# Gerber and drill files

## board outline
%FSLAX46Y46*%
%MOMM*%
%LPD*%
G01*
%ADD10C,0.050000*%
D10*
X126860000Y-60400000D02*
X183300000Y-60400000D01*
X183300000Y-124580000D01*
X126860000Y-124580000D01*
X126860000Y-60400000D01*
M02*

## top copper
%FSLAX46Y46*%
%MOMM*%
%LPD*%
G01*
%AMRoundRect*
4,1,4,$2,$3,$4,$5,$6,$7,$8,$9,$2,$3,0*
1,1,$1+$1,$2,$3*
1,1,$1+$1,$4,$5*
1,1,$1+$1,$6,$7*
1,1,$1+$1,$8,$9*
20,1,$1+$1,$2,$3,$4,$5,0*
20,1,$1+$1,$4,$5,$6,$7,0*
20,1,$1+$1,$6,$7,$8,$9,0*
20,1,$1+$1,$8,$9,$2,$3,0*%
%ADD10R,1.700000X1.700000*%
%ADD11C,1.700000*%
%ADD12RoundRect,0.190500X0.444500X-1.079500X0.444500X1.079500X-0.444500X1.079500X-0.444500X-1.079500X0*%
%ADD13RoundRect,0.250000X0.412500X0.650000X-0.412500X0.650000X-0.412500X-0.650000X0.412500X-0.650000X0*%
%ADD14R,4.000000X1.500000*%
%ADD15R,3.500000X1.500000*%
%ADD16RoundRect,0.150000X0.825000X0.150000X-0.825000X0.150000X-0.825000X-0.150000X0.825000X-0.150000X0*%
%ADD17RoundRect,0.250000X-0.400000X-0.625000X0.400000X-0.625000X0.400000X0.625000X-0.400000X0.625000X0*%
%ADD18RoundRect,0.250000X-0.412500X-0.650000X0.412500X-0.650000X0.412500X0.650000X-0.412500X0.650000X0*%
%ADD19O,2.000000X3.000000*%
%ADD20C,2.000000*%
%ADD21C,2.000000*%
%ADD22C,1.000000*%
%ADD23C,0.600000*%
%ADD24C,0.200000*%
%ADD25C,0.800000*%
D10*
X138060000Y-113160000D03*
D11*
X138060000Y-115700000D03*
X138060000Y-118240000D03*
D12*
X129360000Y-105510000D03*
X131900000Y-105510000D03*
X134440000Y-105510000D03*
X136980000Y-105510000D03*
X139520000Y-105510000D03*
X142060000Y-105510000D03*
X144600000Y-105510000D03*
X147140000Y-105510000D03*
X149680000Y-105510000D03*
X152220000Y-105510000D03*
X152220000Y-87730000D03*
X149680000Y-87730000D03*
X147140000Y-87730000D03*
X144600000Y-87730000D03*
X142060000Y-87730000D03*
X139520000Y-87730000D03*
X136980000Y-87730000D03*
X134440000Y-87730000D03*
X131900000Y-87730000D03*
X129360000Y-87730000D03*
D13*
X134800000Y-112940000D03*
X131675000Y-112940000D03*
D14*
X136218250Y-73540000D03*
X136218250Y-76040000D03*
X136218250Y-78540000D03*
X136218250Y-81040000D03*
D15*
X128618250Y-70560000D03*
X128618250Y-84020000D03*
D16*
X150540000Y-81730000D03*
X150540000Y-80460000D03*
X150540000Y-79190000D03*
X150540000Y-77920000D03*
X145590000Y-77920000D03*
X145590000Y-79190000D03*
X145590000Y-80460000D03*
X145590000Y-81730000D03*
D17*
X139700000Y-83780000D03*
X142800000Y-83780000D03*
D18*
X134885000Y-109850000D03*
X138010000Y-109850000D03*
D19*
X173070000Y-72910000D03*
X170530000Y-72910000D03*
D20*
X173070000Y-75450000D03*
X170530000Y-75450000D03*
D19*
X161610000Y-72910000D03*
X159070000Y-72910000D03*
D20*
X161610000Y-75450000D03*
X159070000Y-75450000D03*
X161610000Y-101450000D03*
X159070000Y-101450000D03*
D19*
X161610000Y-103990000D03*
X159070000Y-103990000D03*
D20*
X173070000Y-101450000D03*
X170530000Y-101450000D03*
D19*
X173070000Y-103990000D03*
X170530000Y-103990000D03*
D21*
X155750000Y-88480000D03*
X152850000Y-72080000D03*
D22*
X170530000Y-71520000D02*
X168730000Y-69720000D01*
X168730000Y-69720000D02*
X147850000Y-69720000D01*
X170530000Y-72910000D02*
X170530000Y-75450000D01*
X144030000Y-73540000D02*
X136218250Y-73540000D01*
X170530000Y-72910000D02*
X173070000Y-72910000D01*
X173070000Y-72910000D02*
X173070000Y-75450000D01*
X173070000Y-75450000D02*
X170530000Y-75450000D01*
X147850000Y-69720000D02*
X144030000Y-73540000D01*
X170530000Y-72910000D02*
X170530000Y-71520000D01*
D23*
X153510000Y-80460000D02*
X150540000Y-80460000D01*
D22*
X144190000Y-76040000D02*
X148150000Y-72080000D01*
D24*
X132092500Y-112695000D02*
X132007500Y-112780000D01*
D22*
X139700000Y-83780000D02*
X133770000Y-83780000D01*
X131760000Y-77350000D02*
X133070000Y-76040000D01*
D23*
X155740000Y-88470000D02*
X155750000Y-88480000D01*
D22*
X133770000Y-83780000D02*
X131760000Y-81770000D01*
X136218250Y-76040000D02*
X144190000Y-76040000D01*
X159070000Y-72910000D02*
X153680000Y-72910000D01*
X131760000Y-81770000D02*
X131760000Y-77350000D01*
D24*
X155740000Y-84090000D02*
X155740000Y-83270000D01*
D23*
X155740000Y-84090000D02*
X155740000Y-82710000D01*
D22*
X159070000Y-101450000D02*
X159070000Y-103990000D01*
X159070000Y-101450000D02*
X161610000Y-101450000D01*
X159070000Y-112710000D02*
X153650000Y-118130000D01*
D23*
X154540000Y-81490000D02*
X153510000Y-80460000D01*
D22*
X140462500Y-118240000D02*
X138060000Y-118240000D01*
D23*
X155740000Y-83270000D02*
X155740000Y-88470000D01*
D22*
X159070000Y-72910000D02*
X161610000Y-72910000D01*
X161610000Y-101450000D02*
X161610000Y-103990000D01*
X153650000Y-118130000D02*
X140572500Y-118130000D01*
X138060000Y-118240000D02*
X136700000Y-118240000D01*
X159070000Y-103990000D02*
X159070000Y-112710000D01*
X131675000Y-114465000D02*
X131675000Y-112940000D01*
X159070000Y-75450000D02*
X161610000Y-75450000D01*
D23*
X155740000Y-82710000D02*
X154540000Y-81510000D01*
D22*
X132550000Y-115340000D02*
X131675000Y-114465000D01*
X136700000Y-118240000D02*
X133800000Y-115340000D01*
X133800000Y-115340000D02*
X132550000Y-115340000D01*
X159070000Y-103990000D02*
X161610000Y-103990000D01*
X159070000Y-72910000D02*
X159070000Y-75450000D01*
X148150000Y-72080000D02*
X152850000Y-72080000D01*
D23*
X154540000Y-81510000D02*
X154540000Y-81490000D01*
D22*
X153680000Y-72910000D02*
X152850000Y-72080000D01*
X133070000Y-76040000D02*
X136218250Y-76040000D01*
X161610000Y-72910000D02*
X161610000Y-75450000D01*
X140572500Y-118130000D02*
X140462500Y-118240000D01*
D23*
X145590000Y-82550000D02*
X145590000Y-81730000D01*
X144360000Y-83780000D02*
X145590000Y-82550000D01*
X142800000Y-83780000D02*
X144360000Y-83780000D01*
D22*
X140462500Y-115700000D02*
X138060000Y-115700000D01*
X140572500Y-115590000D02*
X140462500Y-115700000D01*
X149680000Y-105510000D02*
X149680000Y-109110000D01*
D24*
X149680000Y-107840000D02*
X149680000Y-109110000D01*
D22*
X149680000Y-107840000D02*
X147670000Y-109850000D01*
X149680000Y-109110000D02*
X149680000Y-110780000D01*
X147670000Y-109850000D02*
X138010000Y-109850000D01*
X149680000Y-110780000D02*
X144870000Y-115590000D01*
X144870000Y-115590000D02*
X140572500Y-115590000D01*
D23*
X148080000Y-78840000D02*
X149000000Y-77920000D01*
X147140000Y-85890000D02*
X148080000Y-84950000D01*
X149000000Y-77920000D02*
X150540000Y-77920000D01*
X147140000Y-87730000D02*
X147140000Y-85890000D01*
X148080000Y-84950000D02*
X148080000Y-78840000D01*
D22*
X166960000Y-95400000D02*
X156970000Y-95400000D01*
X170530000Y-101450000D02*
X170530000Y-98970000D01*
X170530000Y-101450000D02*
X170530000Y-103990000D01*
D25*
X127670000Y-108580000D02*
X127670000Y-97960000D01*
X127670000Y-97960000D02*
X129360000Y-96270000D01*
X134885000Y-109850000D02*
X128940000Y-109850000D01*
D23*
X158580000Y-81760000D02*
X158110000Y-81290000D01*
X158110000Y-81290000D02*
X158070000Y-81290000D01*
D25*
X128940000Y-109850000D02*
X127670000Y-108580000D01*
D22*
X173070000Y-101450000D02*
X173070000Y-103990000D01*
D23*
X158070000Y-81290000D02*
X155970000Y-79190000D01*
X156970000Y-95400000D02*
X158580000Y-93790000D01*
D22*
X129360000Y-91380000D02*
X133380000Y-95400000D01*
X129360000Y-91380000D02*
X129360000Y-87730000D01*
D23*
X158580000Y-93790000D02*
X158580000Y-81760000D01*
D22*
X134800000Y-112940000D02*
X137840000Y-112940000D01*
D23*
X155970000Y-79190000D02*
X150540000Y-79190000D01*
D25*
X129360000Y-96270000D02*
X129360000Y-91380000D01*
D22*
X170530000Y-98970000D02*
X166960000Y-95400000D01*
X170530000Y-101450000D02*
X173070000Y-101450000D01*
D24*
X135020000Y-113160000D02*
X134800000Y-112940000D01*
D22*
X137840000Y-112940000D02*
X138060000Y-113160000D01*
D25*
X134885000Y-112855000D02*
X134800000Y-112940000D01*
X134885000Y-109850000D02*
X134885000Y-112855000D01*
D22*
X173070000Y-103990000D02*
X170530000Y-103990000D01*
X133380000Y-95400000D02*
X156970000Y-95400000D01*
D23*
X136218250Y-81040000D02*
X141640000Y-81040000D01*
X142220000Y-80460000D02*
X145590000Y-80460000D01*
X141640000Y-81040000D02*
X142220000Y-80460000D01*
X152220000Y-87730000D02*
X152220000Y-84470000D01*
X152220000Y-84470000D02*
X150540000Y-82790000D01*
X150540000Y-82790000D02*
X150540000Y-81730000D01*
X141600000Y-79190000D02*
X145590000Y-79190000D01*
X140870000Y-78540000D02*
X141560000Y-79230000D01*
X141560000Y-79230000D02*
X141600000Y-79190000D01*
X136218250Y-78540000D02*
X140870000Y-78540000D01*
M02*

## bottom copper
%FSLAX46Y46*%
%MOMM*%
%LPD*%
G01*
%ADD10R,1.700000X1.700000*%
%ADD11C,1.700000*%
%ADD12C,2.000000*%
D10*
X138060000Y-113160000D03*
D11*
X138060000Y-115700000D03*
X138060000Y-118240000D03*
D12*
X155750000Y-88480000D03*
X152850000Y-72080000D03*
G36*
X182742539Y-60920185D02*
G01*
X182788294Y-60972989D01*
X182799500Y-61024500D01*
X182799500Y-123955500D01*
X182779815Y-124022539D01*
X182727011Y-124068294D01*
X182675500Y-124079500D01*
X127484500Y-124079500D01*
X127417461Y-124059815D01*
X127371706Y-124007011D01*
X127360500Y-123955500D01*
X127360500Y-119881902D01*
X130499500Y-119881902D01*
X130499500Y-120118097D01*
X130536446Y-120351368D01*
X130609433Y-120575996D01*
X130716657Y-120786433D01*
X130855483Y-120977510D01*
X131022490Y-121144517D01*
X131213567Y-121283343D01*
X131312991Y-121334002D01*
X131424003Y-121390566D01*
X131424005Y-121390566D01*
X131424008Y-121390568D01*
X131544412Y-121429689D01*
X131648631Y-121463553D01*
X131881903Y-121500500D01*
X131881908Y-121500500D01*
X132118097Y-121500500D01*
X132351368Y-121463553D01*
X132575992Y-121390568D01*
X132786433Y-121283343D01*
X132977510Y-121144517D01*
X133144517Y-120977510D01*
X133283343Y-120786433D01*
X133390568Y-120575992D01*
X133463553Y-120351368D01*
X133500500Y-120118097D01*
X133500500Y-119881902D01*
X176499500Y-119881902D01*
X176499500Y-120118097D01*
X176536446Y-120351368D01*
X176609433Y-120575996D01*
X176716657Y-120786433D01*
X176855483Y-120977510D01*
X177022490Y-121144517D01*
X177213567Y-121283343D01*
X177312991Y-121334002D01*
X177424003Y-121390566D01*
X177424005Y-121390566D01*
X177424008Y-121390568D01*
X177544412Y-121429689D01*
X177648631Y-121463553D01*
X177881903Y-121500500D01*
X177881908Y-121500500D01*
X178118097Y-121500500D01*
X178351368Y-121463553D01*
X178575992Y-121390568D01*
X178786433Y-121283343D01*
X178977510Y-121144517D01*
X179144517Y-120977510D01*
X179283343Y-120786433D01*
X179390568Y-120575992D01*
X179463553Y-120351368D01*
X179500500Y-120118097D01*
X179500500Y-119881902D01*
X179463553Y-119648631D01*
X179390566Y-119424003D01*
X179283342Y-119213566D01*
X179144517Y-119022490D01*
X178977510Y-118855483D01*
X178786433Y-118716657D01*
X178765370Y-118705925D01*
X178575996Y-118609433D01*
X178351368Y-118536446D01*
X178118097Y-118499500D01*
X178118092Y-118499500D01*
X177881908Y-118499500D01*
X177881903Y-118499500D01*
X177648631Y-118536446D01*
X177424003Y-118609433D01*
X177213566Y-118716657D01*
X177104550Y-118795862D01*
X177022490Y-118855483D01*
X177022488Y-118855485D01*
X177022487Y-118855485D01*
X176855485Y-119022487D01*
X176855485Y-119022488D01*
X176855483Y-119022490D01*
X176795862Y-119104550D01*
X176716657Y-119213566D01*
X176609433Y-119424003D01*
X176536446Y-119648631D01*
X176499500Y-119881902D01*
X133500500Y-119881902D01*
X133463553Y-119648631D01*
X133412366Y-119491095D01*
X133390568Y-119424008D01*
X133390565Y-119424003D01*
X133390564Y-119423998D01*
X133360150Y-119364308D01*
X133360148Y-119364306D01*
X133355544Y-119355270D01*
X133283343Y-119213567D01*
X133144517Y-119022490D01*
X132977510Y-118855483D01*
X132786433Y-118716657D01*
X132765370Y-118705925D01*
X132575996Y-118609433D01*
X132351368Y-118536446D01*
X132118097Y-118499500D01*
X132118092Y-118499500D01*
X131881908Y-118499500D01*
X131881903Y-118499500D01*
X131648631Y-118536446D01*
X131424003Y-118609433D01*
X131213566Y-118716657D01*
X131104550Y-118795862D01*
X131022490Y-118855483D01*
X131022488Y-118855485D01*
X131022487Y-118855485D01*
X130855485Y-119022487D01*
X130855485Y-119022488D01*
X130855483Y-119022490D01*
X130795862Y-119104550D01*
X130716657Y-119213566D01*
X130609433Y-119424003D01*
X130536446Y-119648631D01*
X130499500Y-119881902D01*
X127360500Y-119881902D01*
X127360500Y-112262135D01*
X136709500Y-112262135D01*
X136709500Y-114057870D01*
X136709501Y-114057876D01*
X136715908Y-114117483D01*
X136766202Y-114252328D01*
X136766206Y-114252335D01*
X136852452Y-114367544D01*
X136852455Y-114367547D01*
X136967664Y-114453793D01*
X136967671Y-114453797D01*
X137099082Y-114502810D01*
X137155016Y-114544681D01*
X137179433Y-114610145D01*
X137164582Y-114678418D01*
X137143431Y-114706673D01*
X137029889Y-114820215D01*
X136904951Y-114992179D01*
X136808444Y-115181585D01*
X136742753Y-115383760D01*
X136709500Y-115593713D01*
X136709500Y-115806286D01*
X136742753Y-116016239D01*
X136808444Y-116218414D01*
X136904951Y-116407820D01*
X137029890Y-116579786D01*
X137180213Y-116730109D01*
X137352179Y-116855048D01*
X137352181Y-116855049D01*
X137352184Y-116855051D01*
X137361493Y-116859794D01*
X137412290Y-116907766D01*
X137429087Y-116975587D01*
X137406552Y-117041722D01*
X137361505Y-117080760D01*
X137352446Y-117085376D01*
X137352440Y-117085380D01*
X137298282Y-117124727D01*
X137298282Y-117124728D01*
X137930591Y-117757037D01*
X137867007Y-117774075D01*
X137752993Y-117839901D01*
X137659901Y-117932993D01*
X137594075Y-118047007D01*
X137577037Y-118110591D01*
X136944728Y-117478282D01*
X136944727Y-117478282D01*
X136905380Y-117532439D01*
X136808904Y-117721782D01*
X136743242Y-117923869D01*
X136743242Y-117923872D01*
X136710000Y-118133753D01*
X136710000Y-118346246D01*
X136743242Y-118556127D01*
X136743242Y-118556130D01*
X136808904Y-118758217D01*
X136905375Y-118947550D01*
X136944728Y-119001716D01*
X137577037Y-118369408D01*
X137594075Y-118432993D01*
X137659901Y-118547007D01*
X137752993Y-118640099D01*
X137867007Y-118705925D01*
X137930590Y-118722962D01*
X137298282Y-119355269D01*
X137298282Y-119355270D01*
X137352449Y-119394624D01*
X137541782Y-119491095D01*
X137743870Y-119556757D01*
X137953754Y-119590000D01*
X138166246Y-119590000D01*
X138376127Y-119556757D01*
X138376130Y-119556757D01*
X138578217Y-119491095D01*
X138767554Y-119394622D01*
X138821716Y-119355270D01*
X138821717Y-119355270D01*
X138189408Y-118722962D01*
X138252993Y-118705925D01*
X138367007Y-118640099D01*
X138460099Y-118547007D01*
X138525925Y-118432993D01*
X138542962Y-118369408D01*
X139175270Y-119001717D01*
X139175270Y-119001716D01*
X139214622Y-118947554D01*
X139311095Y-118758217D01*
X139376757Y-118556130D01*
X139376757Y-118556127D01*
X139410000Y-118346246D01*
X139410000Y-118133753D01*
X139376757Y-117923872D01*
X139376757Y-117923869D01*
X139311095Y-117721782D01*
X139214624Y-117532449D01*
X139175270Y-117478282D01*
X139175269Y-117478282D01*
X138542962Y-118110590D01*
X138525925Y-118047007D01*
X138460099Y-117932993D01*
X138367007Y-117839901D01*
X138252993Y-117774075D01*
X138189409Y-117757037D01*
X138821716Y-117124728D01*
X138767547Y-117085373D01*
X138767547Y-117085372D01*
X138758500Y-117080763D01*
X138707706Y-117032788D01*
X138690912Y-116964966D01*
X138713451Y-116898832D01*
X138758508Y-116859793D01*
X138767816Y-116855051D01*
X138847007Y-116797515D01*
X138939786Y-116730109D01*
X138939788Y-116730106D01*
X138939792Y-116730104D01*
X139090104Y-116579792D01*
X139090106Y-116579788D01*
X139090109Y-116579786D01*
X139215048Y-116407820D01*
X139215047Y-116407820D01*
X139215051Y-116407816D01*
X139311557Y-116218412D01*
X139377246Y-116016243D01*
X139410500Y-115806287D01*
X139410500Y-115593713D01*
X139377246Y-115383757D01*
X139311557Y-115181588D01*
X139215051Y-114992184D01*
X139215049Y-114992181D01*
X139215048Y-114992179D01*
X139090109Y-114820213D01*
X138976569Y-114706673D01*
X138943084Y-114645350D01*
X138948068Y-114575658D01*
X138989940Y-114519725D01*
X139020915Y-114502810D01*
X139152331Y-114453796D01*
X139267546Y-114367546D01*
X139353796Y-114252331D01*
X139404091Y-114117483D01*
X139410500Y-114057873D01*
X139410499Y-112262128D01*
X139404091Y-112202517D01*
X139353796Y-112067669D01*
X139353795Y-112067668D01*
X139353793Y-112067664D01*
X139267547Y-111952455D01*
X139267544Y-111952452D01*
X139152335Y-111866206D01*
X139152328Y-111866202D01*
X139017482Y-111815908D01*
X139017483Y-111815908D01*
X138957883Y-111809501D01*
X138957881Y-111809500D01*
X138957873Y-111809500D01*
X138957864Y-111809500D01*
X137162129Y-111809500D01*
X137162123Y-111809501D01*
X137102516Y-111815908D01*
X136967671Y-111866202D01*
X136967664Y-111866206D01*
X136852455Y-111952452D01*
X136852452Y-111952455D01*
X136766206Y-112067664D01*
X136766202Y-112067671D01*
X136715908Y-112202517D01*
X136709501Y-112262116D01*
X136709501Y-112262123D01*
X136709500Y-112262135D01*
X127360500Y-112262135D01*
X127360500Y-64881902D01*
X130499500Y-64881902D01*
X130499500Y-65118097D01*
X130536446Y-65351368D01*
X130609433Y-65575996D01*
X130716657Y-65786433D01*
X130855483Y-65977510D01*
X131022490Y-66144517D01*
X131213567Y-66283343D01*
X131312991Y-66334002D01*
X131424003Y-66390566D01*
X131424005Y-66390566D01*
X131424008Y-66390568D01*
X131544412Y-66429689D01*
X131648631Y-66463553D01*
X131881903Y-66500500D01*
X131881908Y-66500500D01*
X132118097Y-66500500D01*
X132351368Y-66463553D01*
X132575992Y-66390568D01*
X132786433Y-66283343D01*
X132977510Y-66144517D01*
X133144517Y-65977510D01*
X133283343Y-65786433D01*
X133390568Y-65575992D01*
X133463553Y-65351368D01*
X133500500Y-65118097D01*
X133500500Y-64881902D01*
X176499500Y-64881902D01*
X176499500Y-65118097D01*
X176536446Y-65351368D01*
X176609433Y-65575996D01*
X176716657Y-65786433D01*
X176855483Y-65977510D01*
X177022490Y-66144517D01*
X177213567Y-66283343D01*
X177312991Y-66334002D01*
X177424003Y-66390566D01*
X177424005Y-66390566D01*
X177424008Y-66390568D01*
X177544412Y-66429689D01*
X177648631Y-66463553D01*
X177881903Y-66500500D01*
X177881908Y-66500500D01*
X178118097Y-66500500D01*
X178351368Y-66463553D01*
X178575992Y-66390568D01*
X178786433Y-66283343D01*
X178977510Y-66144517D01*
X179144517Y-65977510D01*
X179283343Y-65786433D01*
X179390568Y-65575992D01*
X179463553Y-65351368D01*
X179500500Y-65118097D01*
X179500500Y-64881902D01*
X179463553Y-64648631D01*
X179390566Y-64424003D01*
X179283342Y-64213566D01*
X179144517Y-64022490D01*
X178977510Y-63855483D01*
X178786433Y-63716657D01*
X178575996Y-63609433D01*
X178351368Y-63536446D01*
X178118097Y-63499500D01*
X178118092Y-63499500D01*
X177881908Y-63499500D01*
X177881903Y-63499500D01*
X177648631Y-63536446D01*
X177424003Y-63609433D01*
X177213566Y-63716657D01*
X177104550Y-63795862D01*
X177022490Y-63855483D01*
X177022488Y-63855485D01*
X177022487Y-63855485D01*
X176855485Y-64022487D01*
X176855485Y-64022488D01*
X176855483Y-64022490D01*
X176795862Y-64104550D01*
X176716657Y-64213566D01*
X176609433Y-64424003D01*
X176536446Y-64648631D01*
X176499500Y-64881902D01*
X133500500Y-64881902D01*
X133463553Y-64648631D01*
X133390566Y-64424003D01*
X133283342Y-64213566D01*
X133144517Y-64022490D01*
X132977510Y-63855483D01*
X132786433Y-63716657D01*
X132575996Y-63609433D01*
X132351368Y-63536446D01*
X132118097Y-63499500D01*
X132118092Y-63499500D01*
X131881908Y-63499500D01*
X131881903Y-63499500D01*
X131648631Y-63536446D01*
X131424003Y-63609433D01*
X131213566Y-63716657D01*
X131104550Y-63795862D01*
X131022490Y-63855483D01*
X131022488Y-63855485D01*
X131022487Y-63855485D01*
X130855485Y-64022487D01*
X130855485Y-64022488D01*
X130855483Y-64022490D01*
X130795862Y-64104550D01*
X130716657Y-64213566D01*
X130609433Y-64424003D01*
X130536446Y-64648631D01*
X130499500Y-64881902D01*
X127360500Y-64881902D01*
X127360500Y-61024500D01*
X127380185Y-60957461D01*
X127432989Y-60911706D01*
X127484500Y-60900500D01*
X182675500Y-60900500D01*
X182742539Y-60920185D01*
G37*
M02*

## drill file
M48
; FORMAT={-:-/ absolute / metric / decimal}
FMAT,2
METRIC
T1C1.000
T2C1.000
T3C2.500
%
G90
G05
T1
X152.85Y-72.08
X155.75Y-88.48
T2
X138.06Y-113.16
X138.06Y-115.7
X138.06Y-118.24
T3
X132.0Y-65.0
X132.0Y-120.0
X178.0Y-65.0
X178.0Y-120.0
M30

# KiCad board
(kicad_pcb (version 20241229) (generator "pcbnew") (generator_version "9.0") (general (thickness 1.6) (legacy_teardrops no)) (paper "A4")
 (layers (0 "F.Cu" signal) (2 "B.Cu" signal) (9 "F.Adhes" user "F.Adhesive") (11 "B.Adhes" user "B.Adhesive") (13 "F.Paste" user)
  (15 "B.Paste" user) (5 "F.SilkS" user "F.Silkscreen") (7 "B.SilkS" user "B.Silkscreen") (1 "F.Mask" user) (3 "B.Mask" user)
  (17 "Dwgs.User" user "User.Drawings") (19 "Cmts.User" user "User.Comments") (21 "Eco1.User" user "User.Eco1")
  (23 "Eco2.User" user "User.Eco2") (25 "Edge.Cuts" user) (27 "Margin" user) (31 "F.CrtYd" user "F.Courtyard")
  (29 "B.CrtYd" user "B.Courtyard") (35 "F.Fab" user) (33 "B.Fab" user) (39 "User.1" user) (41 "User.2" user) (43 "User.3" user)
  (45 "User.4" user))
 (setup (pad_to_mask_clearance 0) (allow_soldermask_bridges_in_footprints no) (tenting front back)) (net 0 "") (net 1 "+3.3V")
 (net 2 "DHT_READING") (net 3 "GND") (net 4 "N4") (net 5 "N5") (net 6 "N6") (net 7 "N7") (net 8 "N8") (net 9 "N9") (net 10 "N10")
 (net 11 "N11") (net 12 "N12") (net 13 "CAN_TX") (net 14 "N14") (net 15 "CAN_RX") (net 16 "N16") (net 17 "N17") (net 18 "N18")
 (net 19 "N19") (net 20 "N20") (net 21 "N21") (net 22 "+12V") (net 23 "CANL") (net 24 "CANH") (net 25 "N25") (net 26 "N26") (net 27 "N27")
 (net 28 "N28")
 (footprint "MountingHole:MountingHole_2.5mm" (layer "F.Cu") (at 178 65)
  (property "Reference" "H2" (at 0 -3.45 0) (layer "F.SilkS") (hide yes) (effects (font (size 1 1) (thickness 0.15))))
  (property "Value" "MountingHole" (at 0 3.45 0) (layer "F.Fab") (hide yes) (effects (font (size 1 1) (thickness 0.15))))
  (pad "" np_thru_hole circle (at 0 0) (size 2.5 2.5) (drill 2.5) (layers "*.Cu" "*.Mask")))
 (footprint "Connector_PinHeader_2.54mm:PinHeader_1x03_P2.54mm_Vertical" (layer "F.Cu") (at 138.06 113.16)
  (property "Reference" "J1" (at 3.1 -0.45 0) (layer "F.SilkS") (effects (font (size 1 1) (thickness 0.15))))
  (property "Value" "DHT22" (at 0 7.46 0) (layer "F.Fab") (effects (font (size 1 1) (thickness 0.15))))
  (pad "1" thru_hole rect (at 0 0) (size 1.7 1.7) (drill 1) (layers "*.Cu" "*.Mask") (remove_unused_layers no) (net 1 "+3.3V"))
  (pad "2" thru_hole circle (at 0 2.54) (size 1.7 1.7) (drill 1) (layers "*.Cu" "*.Mask") (remove_unused_layers no) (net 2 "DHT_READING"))
  (pad "3" thru_hole circle (at 0 5.08) (size 1.7 1.7) (drill 1) (layers "*.Cu" "*.Mask") (remove_unused_layers no) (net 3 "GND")))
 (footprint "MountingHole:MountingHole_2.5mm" (layer "F.Cu") (at 132 65)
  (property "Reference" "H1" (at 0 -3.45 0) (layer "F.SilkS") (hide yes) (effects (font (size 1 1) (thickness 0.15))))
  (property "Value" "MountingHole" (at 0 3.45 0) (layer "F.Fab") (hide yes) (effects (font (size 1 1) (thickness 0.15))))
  (pad "" np_thru_hole circle (at 0 0) (size 2.5 2.5) (drill 2.5) (layers "*.Cu" "*.Mask")))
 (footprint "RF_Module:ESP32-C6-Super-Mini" (layer "F.Cu") (at 157.338 110.165 90)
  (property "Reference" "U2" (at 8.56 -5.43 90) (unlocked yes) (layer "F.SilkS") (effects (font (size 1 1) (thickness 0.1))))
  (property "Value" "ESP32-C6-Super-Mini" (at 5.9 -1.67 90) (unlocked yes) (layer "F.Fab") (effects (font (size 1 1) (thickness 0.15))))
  (pad "1" smd roundrect (at 4.655 -27.978 90) (size 2.54 1.27) (layers "F.Cu" "F.Mask" "F.Paste") (roundrect_rratio 0.15) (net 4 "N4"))
  (pad "2" smd roundrect (at 4.655 -25.438 90) (size 2.54 1.27) (layers "F.Cu" "F.Mask" "F.Paste") (roundrect_rratio 0.15) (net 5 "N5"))
  (pad "3" smd roundrect (at 4.655 -22.898 90) (size 2.54 1.27) (layers "F.Cu" "F.Mask" "F.Paste") (roundrect_rratio 0.15) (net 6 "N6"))
  (pad "4" smd roundrect (at 4.655 -20.358 90) (size 2.54 1.27) (layers "F.Cu" "F.Mask" "F.Paste") (roundrect_rratio 0.15) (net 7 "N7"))
  (pad "5" smd roundrect (at 4.655 -17.818 90) (size 2.54 1.27) (layers "F.Cu" "F.Mask" "F.Paste") (roundrect_rratio 0.15) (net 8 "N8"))
  (pad "6" smd roundrect (at 4.655 -15.278 90) (size 2.54 1.27) (layers "F.Cu" "F.Mask" "F.Paste") (roundrect_rratio 0.15) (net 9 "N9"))
  (pad "7" smd roundrect (at 4.655 -12.738 90) (size 2.54 1.27) (layers "F.Cu" "F.Mask" "F.Paste") (roundrect_rratio 0.15) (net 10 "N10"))
  (pad "8" smd roundrect (at 4.655 -10.198 90) (size 2.54 1.27) (layers "F.Cu" "F.Mask" "F.Paste") (roundrect_rratio 0.15) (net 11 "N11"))
  (pad "9" smd roundrect (at 4.655 -7.658 90) (size 2.54 1.27) (layers "F.Cu" "F.Mask" "F.Paste") (roundrect_rratio 0.15)
   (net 2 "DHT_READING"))
  (pad "10" smd roundrect (at 4.655 -5.118 90) (size 2.54 1.27) (layers "F.Cu" "F.Mask" "F.Paste") (roundrect_rratio 0.15) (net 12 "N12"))
  (pad "11" smd roundrect (at 22.435 -5.118 90) (size 2.54 1.27) (layers "F.Cu" "F.Mask" "F.Paste") (roundrect_rratio 0.15)
   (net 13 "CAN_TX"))
  (pad "12" smd roundrect (at 22.435 -7.658 90) (size 2.54 1.27) (layers "F.Cu" "F.Mask" "F.Paste") (roundrect_rratio 0.15) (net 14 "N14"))
  (pad "13" smd roundrect (at 22.435 -10.198 90) (size 2.54 1.27) (layers "F.Cu" "F.Mask" "F.Paste") (roundrect_rratio 0.15)
   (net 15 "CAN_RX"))
  (pad "14" smd roundrect (at 22.435 -12.738 90) (size 2.54 1.27) (layers "F.Cu" "F.Mask" "F.Paste") (roundrect_rratio 0.15) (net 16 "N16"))
  (pad "15" smd roundrect (at 22.435 -15.278 90) (size 2.54 1.27) (layers "F.Cu" "F.Mask" "F.Paste") (roundrect_rratio 0.15) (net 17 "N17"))
  (pad "16" smd roundrect (at 22.435 -17.818 90) (size 2.54 1.27) (layers "F.Cu" "F.Mask" "F.Paste") (roundrect_rratio 0.15) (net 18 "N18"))
  (pad "17" smd roundrect (at 22.435 -20.358 90) (size 2.54 1.27) (layers "F.Cu" "F.Mask" "F.Paste") (roundrect_rratio 0.15) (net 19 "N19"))
  (pad "18" smd roundrect (at 22.435 -22.898 90) (size 2.54 1.27) (layers "F.Cu" "F.Mask" "F.Paste") (roundrect_rratio 0.15) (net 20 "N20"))
  (pad "19" smd roundrect (at 22.435 -25.438 90) (size 2.54 1.27) (layers "F.Cu" "F.Mask" "F.Paste") (roundrect_rratio 0.15) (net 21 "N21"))
  (pad "20" smd roundrect (at 22.435 -27.978 90) (size 2.54 1.27) (layers "F.Cu" "F.Mask" "F.Paste") (roundrect_rratio 0.15) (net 1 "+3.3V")))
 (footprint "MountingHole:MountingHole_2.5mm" (layer "F.Cu") (at 132 120)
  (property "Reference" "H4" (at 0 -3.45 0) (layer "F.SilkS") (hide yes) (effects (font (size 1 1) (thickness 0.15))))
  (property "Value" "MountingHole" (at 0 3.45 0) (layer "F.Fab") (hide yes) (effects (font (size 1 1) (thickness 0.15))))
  (pad "" np_thru_hole circle (at 0 0) (size 2.5 2.5) (drill 2.5) (layers "*.Cu" "*.Mask")))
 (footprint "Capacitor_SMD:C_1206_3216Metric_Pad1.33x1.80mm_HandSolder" (layer "F.Cu") (at 133.2375 112.94 180)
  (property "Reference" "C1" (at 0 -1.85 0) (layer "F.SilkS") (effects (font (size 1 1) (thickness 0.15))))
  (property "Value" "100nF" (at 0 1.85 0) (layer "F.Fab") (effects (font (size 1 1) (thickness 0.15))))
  (pad "1" smd roundrect (at -1.5625 0 180) (size 1.325 1.8) (layers "F.Cu" "F.Mask" "F.Paste") (roundrect_rratio 0.188679) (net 1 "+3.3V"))
  (pad "2" smd roundrect (at 1.5625 0 180) (size 1.325 1.8) (layers "F.Cu" "F.Mask" "F.Paste") (roundrect_rratio 0.188679) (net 3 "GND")))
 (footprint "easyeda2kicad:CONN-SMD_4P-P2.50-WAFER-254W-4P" (layer "F.Cu") (at 132.41825 77.29 -90)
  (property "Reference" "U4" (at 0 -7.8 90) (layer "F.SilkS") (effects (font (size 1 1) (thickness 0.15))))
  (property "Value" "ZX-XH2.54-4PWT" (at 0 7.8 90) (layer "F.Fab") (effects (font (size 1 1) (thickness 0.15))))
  (pad "1" smd rect (at -3.75 -3.8 270) (size 1.5 4) (layers "F.Cu" "F.Mask" "F.Paste") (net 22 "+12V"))
  (pad "2" smd rect (at -1.25 -3.8 270) (size 1.5 4) (layers "F.Cu" "F.Mask" "F.Paste") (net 3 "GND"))
  (pad "3" smd rect (at 1.25 -3.8 270) (size 1.5 4) (layers "F.Cu" "F.Mask" "F.Paste") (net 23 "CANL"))
  (pad "4" smd rect (at 3.75 -3.8 270) (size 1.5 4) (layers "F.Cu" "F.Mask" "F.Paste") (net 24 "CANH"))
  (pad "5" smd rect (at -6.73 3.8 270) (size 1.5 3.5) (layers "F.Cu" "F.Mask" "F.Paste") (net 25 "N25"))
  (pad "6" smd rect (at 6.73 3.8 270) (size 1.5 3.5) (layers "F.Cu" "F.Mask" "F.Paste") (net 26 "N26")))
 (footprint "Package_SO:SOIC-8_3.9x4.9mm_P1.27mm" (layer "F.Cu") (at 148.065 79.825 180)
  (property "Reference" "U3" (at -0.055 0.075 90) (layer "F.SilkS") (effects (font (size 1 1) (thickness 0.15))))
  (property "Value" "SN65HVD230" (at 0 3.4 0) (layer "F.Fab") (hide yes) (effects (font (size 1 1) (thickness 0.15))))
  (pad "1" smd roundrect (at -2.475 -1.905 180) (size 1.95 0.6) (layers "F.Cu" "F.Mask" "F.Paste") (roundrect_rratio 0.25) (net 13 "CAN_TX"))
  (pad "2" smd roundrect (at -2.475 -0.635 180) (size 1.95 0.6) (layers "F.Cu" "F.Mask" "F.Paste") (roundrect_rratio 0.25) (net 3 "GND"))
  (pad "3" smd roundrect (at -2.475 0.635 180) (size 1.95 0.6) (layers "F.Cu" "F.Mask" "F.Paste") (roundrect_rratio 0.25) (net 1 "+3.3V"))
  (pad "4" smd roundrect (at -2.475 1.905 180) (size 1.95 0.6) (layers "F.Cu" "F.Mask" "F.Paste") (roundrect_rratio 0.25) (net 15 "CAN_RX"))
  (pad "5" smd roundrect (at 2.475 1.905 180) (size 1.95 0.6) (layers "F.Cu" "F.Mask" "F.Paste") (roundrect_rratio 0.25) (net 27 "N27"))
  (pad "6" smd roundrect (at 2.475 0.635 180) (size 1.95 0.6) (layers "F.Cu" "F.Mask" "F.Paste") (roundrect_rratio 0.25) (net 23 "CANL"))
  (pad "7" smd roundrect (at 2.475 -0.635 180) (size 1.95 0.6) (layers "F.Cu" "F.Mask" "F.Paste") (roundrect_rratio 0.25) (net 24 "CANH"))
  (pad "8" smd roundrect (at 2.475 -1.905 180) (size 1.95 0.6) (layers "F.Cu" "F.Mask" "F.Paste") (roundrect_rratio 0.25) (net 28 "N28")))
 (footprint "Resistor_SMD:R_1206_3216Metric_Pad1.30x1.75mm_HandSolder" (layer "F.Cu") (at 141.25 83.78)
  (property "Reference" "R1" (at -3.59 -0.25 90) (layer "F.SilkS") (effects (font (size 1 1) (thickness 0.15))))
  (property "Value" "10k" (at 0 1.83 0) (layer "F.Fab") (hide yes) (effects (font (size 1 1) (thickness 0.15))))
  (pad "1" smd roundrect (at -1.55 0) (size 1.3 1.75) (layers "F.Cu" "F.Mask" "F.Paste") (roundrect_rratio 0.192308) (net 3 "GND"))
  (pad "2" smd roundrect (at 1.55 0) (size 1.3 1.75) (layers "F.Cu" "F.Mask" "F.Paste") (roundrect_rratio 0.192308) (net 28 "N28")))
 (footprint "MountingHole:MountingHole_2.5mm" (layer "F.Cu") (at 178 120)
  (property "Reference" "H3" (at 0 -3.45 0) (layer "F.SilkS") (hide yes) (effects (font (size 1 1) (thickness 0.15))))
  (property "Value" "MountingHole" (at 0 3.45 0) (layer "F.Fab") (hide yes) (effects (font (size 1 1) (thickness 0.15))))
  (pad "" np_thru_hole circle (at 0 0) (size 2.5 2.5) (drill 2.5) (layers "*.Cu" "*.Mask")))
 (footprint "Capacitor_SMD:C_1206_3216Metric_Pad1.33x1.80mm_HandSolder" (layer "F.Cu") (at 136.4475 109.85)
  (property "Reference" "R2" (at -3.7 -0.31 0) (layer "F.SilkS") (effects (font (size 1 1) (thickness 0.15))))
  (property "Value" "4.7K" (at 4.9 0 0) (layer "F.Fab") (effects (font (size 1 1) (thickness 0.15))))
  (pad "1" smd roundrect (at -1.5625 0) (size 1.325 1.8) (layers "F.Cu" "F.Mask" "F.Paste") (roundrect_rratio 0.188679) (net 1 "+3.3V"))
  (pad "2" smd roundrect (at 1.5625 0) (size 1.325 1.8) (layers "F.Cu" "F.Mask" "F.Paste") (roundrect_rratio 0.188679) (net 2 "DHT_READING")))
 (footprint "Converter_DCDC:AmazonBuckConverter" (layer "F.Cu") (at 153.99 75.45 -90)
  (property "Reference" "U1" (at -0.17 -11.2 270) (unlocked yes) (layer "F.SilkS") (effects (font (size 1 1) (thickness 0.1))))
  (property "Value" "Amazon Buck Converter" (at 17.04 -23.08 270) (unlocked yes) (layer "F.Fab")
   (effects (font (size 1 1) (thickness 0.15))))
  (pad "1" smd oval (at -2.54 -19.08) (size 2 3) (layers "F.Cu" "F.Mask" "F.Paste") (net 22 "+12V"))
  (pad "1" smd oval (at -2.54 -16.54) (size 2 3) (layers "F.Cu" "F.Mask" "F.Paste") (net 22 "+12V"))
  (pad "1" smd circle (at 0 -19.08) (size 2 2) (layers "F.Cu" "F.Mask" "F.Paste") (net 22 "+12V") (thermal_bridge_angle 90))
  (pad "1" smd circle (at 0 -16.54) (size 2 2) (layers "F.Cu" "F.Mask" "F.Paste") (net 22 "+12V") (thermal_bridge_angle 90))
  (pad "2" smd oval (at -2.54 -7.62) (size 2 3) (layers "F.Cu" "F.Mask" "F.Paste") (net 3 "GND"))
  (pad "2" smd oval (at -2.54 -5.08) (size 2 3) (layers "F.Cu" "F.Mask" "F.Paste") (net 3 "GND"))
  (pad "2" smd circle (at 0 -7.62) (size 2 2) (layers "F.Cu" "F.Mask" "F.Paste") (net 3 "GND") (thermal_bridge_angle 90))
  (pad "2" smd circle (at 0 -5.08) (size 2 2) (layers "F.Cu" "F.Mask" "F.Paste") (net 3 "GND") (thermal_bridge_angle 90))
  (pad "3" smd circle (at 26 -7.62) (size 2 2) (layers "F.Cu" "F.Mask" "F.Paste") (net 3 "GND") (thermal_bridge_angle 90))
  (pad "3" smd circle (at 26 -5.08) (size 2 2) (layers "F.Cu" "F.Mask" "F.Paste") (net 3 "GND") (thermal_bridge_angle 90))
  (pad "3" smd oval (at 28.54 -7.62) (size 2 3) (layers "F.Cu" "F.Mask" "F.Paste") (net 3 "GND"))
  (pad "3" smd oval (at 28.54 -5.08) (size 2 3) (layers "F.Cu" "F.Mask" "F.Paste") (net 3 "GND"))
  (pad "4" smd circle (at 26 -19.08) (size 2 2) (layers "F.Cu" "F.Mask" "F.Paste") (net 1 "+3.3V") (thermal_bridge_angle 90))
  (pad "4" smd circle (at 26 -16.54) (size 2 2) (layers "F.Cu" "F.Mask" "F.Paste") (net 1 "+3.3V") (thermal_bridge_angle 90))
  (pad "4" smd oval (at 28.54 -19.08) (size 2 3) (layers "F.Cu" "F.Mask" "F.Paste") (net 1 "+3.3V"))
  (pad "4" smd oval (at 28.54 -16.54) (size 2 3) (layers "F.Cu" "F.Mask" "F.Paste") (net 1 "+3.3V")))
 (gr_rect (start 126.86 60.4) (end 183.3 124.58) (stroke (width 0.05) (type default)) (fill no) (layer "Edge.Cuts"))
 (segment (start 170.53 71.52) (end 168.73 69.72) (width 1) (layer "F.Cu") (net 22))
 (segment (start 168.73 69.72) (end 147.85 69.72) (width 1) (layer "F.Cu") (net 22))
 (segment (start 170.53 72.91) (end 170.53 75.45) (width 1) (layer "F.Cu") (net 22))
 (segment (start 144.03 73.54) (end 136.21825 73.54) (width 1) (layer "F.Cu") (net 22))
 (segment (start 170.53 72.91) (end 173.07 72.91) (width 1) (layer "F.Cu") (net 22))
 (segment (start 173.07 72.91) (end 173.07 75.45) (width 1) (layer "F.Cu") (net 22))
 (segment (start 173.07 75.45) (end 170.53 75.45) (width 1) (layer "F.Cu") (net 22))
 (segment (start 147.85 69.72) (end 144.03 73.54) (width 1) (layer "F.Cu") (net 22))
 (segment (start 170.53 72.91) (end 170.53 71.52) (width 1) (layer "F.Cu") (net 22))
 (segment (start 153.51 80.46) (end 150.54 80.46) (width 0.6) (layer "F.Cu") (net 3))
 (segment (start 144.19 76.04) (end 148.15 72.08) (width 1) (layer "F.Cu") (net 3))
 (segment (start 132.0925 112.695) (end 132.0075 112.78) (width 0.2) (layer "F.Cu") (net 3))
 (segment (start 139.7 83.78) (end 133.77 83.78) (width 1) (layer "F.Cu") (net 3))
 (segment (start 131.76 77.35) (end 133.07 76.04) (width 1) (layer "F.Cu") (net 3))
 (segment (start 155.74 88.47) (end 155.75 88.48) (width 0.6) (layer "F.Cu") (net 3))
 (segment (start 133.77 83.78) (end 131.76 81.77) (width 1) (layer "F.Cu") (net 3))
 (segment (start 136.21825 76.04) (end 144.19 76.04) (width 1) (layer "F.Cu") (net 3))
 (segment (start 159.07 72.91) (end 153.68 72.91) (width 1) (layer "F.Cu") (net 3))
 (segment (start 131.76 81.77) (end 131.76 77.35) (width 1) (layer "F.Cu") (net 3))
 (segment (start 155.74 84.09) (end 155.74 83.27) (width 0.2) (layer "F.Cu") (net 3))
 (segment (start 155.74 84.09) (end 155.74 82.71) (width 0.6) (layer "F.Cu") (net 3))
 (segment (start 159.07 101.45) (end 159.07 103.99) (width 1) (layer "F.Cu") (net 3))
 (segment (start 159.07 101.45) (end 161.61 101.45) (width 1) (layer "F.Cu") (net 3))
 (segment (start 159.07 112.71) (end 153.65 118.13) (width 1) (layer "F.Cu") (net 3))
 (segment (start 154.54 81.49) (end 153.51 80.46) (width 0.6) (layer "F.Cu") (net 3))
 (segment (start 140.4625 118.24) (end 138.06 118.24) (width 1) (layer "F.Cu") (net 3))
 (segment (start 155.74 83.27) (end 155.74 88.47) (width 0.6) (layer "F.Cu") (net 3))
 (segment (start 159.07 72.91) (end 161.61 72.91) (width 1) (layer "F.Cu") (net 3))
 (segment (start 161.61 101.45) (end 161.61 103.99) (width 1) (layer "F.Cu") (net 3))
 (segment (start 153.65 118.13) (end 140.5725 118.13) (width 1) (layer "F.Cu") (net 3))
 (segment (start 138.06 118.24) (end 136.7 118.24) (width 1) (layer "F.Cu") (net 3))
 (segment (start 159.07 103.99) (end 159.07 112.71) (width 1) (layer "F.Cu") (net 3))
 (segment (start 131.675 114.465) (end 131.675 112.94) (width 1) (layer "F.Cu") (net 3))
 (segment (start 159.07 75.45) (end 161.61 75.45) (width 1) (layer "F.Cu") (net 3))
 (segment (start 155.74 82.71) (end 154.54 81.51) (width 0.6) (layer "F.Cu") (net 3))
 (segment (start 132.55 115.34) (end 131.675 114.465) (width 1) (layer "F.Cu") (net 3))
 (segment (start 136.7 118.24) (end 133.8 115.34) (width 1) (layer "F.Cu") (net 3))
 (segment (start 133.8 115.34) (end 132.55 115.34) (width 1) (layer "F.Cu") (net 3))
 (segment (start 159.07 103.99) (end 161.61 103.99) (width 1) (layer "F.Cu") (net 3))
 (segment (start 159.07 72.91) (end 159.07 75.45) (width 1) (layer "F.Cu") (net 3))
 (segment (start 148.15 72.08) (end 152.85 72.08) (width 1) (layer "F.Cu") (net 3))
 (segment (start 154.54 81.51) (end 154.54 81.49) (width 0.6) (layer "F.Cu") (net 3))
 (segment (start 153.68 72.91) (end 152.85 72.08) (width 1) (layer "F.Cu") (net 3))
 (segment (start 133.07 76.04) (end 136.21825 76.04) (width 1) (layer "F.Cu") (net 3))
 (segment (start 161.61 72.91) (end 161.61 75.45) (width 1) (layer "F.Cu") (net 3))
 (segment (start 140.5725 118.13) (end 140.4625 118.24) (width 1) (layer "F.Cu") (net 3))
 (via (at 155.75 88.48) (size 2) (drill 1) (layers "F.Cu" "B.Cu") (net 3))
 (via (at 152.85 72.08) (size 2) (drill 1) (layers "F.Cu" "B.Cu") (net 3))
 (segment (start 145.59 82.55) (end 145.59 81.73) (width 0.6) (layer "F.Cu") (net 28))
 (segment (start 144.36 83.78) (end 145.59 82.55) (width 0.6) (layer "F.Cu") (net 28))
 (segment (start 142.8 83.78) (end 144.36 83.78) (width 0.6) (layer "F.Cu") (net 28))
 (segment (start 140.4625 115.7) (end 138.06 115.7) (width 1) (layer "F.Cu") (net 2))
 (segment (start 140.5725 115.59) (end 140.4625 115.7) (width 1) (layer "F.Cu") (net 2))
 (segment (start 149.68 105.51) (end 149.68 109.11) (width 1) (layer "F.Cu") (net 2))
 (segment (start 149.68 107.84) (end 149.68 109.11) (width 0.2) (layer "F.Cu") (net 2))
 (segment (start 149.68 107.84) (end 147.67 109.85) (width 1) (layer "F.Cu") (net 2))
 (segment (start 149.68 109.11) (end 149.68 110.78) (width 1) (layer "F.Cu") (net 2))
 (segment (start 147.67 109.85) (end 138.01 109.85) (width 1) (layer "F.Cu") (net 2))
 (segment (start 149.68 110.78) (end 144.87 115.59) (width 1) (layer "F.Cu") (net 2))
 (segment (start 144.87 115.59) (end 140.5725 115.59) (width 1) (layer "F.Cu") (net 2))
 (segment (start 148.08 78.84) (end 149 77.92) (width 0.6) (layer "F.Cu") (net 15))
 (segment (start 147.14 85.89) (end 148.08 84.95) (width 0.6) (layer "F.Cu") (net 15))
 (segment (start 149 77.92) (end 150.54 77.92) (width 0.6) (layer "F.Cu") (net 15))
 (segment (start 147.14 87.73) (end 147.14 85.89) (width 0.6) (layer "F.Cu") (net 15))
 (segment (start 148.08 84.95) (end 148.08 78.84) (width 0.6) (layer "F.Cu") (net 15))
 (segment (start 166.96 95.4) (end 156.97 95.4) (width 1) (layer "F.Cu") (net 1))
 (segment (start 170.53 101.45) (end 170.53 98.97) (width 1) (layer "F.Cu") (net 1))
 (segment (start 170.53 101.45) (end 170.53 103.99) (width 1) (layer "F.Cu") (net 1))
 (segment (start 127.67 108.58) (end 127.67 97.96) (width 0.8) (layer "F.Cu") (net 1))
 (segment (start 127.67 97.96) (end 129.36 96.27) (width 0.8) (layer "F.Cu") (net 1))
 (segment (start 134.885 109.85) (end 128.94 109.85) (width 0.8) (layer "F.Cu") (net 1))
 (segment (start 158.58 81.76) (end 158.11 81.29) (width 0.6) (layer "F.Cu") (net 1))
 (segment (start 158.11 81.29) (end 158.07 81.29) (width 0.6) (layer "F.Cu") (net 1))
 (segment (start 128.94 109.85) (end 127.67 108.58) (width 0.8) (layer "F.Cu") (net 1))
 (segment (start 173.07 101.45) (end 173.07 103.99) (width 1) (layer "F.Cu") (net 1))
 (segment (start 158.07 81.29) (end 155.97 79.19) (width 0.6) (layer "F.Cu") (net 1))
 (segment (start 156.97 95.4) (end 158.58 93.79) (width 0.6) (layer "F.Cu") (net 1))
 (segment (start 129.36 91.38) (end 133.38 95.4) (width 1) (layer "F.Cu") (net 1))
 (segment (start 129.36 91.38) (end 129.36 87.73) (width 1) (layer "F.Cu") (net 1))
 (segment (start 158.58 93.79) (end 158.58 81.76) (width 0.6) (layer "F.Cu") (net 1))
 (segment (start 134.8 112.94) (end 137.84 112.94) (width 1) (layer "F.Cu") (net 1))
 (segment (start 155.97 79.19) (end 150.54 79.19) (width 0.6) (layer "F.Cu") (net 1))
 (segment (start 129.36 96.27) (end 129.36 91.38) (width 0.8) (layer "F.Cu") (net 1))
 (segment (start 170.53 98.97) (end 166.96 95.4) (width 1) (layer "F.Cu") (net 1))
 (segment (start 170.53 101.45) (end 173.07 101.45) (width 1) (layer "F.Cu") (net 1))
 (segment (start 135.02 113.16) (end 134.8 112.94) (width 0.2) (layer "F.Cu") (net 1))
 (segment (start 137.84 112.94) (end 138.06 113.16) (width 1) (layer "F.Cu") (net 1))
 (segment (start 134.885 112.855) (end 134.8 112.94) (width 0.8) (layer "F.Cu") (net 1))
 (segment (start 134.885 109.85) (end 134.885 112.855) (width 0.8) (layer "F.Cu") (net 1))
 (segment (start 173.07 103.99) (end 170.53 103.99) (width 1) (layer "F.Cu") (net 1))
 (segment (start 133.38 95.4) (end 156.97 95.4) (width 1) (layer "F.Cu") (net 1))
 (segment (start 136.21825 81.04) (end 141.64 81.04) (width 0.6) (layer "F.Cu") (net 24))
 (segment (start 142.22 80.46) (end 145.59 80.46) (width 0.6) (layer "F.Cu") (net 24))
 (segment (start 141.64 81.04) (end 142.22 80.46) (width 0.6) (layer "F.Cu") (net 24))
 (segment (start 152.22 87.73) (end 152.22 84.47) (width 0.6) (layer "F.Cu") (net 13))
 (segment (start 152.22 84.47) (end 150.54 82.79) (width 0.6) (layer "F.Cu") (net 13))
 (segment (start 150.54 82.79) (end 150.54 81.73) (width 0.6) (layer "F.Cu") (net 13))
 (segment (start 141.6 79.19) (end 145.59 79.19) (width 0.6) (layer "F.Cu") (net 23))
 (segment (start 140.87 78.54) (end 141.56 79.23) (width 0.6) (layer "F.Cu") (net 23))
 (segment (start 141.56 79.23) (end 141.6 79.19) (width 0.6) (layer "F.Cu") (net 23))
 (segment (start 136.21825 78.54) (end 140.87 78.54) (width 0.6) (layer "F.Cu") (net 23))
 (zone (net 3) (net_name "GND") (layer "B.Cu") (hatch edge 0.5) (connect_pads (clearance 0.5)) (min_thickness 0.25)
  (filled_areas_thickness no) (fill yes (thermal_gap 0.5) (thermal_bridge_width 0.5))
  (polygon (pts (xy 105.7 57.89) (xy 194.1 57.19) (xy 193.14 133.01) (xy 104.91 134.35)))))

